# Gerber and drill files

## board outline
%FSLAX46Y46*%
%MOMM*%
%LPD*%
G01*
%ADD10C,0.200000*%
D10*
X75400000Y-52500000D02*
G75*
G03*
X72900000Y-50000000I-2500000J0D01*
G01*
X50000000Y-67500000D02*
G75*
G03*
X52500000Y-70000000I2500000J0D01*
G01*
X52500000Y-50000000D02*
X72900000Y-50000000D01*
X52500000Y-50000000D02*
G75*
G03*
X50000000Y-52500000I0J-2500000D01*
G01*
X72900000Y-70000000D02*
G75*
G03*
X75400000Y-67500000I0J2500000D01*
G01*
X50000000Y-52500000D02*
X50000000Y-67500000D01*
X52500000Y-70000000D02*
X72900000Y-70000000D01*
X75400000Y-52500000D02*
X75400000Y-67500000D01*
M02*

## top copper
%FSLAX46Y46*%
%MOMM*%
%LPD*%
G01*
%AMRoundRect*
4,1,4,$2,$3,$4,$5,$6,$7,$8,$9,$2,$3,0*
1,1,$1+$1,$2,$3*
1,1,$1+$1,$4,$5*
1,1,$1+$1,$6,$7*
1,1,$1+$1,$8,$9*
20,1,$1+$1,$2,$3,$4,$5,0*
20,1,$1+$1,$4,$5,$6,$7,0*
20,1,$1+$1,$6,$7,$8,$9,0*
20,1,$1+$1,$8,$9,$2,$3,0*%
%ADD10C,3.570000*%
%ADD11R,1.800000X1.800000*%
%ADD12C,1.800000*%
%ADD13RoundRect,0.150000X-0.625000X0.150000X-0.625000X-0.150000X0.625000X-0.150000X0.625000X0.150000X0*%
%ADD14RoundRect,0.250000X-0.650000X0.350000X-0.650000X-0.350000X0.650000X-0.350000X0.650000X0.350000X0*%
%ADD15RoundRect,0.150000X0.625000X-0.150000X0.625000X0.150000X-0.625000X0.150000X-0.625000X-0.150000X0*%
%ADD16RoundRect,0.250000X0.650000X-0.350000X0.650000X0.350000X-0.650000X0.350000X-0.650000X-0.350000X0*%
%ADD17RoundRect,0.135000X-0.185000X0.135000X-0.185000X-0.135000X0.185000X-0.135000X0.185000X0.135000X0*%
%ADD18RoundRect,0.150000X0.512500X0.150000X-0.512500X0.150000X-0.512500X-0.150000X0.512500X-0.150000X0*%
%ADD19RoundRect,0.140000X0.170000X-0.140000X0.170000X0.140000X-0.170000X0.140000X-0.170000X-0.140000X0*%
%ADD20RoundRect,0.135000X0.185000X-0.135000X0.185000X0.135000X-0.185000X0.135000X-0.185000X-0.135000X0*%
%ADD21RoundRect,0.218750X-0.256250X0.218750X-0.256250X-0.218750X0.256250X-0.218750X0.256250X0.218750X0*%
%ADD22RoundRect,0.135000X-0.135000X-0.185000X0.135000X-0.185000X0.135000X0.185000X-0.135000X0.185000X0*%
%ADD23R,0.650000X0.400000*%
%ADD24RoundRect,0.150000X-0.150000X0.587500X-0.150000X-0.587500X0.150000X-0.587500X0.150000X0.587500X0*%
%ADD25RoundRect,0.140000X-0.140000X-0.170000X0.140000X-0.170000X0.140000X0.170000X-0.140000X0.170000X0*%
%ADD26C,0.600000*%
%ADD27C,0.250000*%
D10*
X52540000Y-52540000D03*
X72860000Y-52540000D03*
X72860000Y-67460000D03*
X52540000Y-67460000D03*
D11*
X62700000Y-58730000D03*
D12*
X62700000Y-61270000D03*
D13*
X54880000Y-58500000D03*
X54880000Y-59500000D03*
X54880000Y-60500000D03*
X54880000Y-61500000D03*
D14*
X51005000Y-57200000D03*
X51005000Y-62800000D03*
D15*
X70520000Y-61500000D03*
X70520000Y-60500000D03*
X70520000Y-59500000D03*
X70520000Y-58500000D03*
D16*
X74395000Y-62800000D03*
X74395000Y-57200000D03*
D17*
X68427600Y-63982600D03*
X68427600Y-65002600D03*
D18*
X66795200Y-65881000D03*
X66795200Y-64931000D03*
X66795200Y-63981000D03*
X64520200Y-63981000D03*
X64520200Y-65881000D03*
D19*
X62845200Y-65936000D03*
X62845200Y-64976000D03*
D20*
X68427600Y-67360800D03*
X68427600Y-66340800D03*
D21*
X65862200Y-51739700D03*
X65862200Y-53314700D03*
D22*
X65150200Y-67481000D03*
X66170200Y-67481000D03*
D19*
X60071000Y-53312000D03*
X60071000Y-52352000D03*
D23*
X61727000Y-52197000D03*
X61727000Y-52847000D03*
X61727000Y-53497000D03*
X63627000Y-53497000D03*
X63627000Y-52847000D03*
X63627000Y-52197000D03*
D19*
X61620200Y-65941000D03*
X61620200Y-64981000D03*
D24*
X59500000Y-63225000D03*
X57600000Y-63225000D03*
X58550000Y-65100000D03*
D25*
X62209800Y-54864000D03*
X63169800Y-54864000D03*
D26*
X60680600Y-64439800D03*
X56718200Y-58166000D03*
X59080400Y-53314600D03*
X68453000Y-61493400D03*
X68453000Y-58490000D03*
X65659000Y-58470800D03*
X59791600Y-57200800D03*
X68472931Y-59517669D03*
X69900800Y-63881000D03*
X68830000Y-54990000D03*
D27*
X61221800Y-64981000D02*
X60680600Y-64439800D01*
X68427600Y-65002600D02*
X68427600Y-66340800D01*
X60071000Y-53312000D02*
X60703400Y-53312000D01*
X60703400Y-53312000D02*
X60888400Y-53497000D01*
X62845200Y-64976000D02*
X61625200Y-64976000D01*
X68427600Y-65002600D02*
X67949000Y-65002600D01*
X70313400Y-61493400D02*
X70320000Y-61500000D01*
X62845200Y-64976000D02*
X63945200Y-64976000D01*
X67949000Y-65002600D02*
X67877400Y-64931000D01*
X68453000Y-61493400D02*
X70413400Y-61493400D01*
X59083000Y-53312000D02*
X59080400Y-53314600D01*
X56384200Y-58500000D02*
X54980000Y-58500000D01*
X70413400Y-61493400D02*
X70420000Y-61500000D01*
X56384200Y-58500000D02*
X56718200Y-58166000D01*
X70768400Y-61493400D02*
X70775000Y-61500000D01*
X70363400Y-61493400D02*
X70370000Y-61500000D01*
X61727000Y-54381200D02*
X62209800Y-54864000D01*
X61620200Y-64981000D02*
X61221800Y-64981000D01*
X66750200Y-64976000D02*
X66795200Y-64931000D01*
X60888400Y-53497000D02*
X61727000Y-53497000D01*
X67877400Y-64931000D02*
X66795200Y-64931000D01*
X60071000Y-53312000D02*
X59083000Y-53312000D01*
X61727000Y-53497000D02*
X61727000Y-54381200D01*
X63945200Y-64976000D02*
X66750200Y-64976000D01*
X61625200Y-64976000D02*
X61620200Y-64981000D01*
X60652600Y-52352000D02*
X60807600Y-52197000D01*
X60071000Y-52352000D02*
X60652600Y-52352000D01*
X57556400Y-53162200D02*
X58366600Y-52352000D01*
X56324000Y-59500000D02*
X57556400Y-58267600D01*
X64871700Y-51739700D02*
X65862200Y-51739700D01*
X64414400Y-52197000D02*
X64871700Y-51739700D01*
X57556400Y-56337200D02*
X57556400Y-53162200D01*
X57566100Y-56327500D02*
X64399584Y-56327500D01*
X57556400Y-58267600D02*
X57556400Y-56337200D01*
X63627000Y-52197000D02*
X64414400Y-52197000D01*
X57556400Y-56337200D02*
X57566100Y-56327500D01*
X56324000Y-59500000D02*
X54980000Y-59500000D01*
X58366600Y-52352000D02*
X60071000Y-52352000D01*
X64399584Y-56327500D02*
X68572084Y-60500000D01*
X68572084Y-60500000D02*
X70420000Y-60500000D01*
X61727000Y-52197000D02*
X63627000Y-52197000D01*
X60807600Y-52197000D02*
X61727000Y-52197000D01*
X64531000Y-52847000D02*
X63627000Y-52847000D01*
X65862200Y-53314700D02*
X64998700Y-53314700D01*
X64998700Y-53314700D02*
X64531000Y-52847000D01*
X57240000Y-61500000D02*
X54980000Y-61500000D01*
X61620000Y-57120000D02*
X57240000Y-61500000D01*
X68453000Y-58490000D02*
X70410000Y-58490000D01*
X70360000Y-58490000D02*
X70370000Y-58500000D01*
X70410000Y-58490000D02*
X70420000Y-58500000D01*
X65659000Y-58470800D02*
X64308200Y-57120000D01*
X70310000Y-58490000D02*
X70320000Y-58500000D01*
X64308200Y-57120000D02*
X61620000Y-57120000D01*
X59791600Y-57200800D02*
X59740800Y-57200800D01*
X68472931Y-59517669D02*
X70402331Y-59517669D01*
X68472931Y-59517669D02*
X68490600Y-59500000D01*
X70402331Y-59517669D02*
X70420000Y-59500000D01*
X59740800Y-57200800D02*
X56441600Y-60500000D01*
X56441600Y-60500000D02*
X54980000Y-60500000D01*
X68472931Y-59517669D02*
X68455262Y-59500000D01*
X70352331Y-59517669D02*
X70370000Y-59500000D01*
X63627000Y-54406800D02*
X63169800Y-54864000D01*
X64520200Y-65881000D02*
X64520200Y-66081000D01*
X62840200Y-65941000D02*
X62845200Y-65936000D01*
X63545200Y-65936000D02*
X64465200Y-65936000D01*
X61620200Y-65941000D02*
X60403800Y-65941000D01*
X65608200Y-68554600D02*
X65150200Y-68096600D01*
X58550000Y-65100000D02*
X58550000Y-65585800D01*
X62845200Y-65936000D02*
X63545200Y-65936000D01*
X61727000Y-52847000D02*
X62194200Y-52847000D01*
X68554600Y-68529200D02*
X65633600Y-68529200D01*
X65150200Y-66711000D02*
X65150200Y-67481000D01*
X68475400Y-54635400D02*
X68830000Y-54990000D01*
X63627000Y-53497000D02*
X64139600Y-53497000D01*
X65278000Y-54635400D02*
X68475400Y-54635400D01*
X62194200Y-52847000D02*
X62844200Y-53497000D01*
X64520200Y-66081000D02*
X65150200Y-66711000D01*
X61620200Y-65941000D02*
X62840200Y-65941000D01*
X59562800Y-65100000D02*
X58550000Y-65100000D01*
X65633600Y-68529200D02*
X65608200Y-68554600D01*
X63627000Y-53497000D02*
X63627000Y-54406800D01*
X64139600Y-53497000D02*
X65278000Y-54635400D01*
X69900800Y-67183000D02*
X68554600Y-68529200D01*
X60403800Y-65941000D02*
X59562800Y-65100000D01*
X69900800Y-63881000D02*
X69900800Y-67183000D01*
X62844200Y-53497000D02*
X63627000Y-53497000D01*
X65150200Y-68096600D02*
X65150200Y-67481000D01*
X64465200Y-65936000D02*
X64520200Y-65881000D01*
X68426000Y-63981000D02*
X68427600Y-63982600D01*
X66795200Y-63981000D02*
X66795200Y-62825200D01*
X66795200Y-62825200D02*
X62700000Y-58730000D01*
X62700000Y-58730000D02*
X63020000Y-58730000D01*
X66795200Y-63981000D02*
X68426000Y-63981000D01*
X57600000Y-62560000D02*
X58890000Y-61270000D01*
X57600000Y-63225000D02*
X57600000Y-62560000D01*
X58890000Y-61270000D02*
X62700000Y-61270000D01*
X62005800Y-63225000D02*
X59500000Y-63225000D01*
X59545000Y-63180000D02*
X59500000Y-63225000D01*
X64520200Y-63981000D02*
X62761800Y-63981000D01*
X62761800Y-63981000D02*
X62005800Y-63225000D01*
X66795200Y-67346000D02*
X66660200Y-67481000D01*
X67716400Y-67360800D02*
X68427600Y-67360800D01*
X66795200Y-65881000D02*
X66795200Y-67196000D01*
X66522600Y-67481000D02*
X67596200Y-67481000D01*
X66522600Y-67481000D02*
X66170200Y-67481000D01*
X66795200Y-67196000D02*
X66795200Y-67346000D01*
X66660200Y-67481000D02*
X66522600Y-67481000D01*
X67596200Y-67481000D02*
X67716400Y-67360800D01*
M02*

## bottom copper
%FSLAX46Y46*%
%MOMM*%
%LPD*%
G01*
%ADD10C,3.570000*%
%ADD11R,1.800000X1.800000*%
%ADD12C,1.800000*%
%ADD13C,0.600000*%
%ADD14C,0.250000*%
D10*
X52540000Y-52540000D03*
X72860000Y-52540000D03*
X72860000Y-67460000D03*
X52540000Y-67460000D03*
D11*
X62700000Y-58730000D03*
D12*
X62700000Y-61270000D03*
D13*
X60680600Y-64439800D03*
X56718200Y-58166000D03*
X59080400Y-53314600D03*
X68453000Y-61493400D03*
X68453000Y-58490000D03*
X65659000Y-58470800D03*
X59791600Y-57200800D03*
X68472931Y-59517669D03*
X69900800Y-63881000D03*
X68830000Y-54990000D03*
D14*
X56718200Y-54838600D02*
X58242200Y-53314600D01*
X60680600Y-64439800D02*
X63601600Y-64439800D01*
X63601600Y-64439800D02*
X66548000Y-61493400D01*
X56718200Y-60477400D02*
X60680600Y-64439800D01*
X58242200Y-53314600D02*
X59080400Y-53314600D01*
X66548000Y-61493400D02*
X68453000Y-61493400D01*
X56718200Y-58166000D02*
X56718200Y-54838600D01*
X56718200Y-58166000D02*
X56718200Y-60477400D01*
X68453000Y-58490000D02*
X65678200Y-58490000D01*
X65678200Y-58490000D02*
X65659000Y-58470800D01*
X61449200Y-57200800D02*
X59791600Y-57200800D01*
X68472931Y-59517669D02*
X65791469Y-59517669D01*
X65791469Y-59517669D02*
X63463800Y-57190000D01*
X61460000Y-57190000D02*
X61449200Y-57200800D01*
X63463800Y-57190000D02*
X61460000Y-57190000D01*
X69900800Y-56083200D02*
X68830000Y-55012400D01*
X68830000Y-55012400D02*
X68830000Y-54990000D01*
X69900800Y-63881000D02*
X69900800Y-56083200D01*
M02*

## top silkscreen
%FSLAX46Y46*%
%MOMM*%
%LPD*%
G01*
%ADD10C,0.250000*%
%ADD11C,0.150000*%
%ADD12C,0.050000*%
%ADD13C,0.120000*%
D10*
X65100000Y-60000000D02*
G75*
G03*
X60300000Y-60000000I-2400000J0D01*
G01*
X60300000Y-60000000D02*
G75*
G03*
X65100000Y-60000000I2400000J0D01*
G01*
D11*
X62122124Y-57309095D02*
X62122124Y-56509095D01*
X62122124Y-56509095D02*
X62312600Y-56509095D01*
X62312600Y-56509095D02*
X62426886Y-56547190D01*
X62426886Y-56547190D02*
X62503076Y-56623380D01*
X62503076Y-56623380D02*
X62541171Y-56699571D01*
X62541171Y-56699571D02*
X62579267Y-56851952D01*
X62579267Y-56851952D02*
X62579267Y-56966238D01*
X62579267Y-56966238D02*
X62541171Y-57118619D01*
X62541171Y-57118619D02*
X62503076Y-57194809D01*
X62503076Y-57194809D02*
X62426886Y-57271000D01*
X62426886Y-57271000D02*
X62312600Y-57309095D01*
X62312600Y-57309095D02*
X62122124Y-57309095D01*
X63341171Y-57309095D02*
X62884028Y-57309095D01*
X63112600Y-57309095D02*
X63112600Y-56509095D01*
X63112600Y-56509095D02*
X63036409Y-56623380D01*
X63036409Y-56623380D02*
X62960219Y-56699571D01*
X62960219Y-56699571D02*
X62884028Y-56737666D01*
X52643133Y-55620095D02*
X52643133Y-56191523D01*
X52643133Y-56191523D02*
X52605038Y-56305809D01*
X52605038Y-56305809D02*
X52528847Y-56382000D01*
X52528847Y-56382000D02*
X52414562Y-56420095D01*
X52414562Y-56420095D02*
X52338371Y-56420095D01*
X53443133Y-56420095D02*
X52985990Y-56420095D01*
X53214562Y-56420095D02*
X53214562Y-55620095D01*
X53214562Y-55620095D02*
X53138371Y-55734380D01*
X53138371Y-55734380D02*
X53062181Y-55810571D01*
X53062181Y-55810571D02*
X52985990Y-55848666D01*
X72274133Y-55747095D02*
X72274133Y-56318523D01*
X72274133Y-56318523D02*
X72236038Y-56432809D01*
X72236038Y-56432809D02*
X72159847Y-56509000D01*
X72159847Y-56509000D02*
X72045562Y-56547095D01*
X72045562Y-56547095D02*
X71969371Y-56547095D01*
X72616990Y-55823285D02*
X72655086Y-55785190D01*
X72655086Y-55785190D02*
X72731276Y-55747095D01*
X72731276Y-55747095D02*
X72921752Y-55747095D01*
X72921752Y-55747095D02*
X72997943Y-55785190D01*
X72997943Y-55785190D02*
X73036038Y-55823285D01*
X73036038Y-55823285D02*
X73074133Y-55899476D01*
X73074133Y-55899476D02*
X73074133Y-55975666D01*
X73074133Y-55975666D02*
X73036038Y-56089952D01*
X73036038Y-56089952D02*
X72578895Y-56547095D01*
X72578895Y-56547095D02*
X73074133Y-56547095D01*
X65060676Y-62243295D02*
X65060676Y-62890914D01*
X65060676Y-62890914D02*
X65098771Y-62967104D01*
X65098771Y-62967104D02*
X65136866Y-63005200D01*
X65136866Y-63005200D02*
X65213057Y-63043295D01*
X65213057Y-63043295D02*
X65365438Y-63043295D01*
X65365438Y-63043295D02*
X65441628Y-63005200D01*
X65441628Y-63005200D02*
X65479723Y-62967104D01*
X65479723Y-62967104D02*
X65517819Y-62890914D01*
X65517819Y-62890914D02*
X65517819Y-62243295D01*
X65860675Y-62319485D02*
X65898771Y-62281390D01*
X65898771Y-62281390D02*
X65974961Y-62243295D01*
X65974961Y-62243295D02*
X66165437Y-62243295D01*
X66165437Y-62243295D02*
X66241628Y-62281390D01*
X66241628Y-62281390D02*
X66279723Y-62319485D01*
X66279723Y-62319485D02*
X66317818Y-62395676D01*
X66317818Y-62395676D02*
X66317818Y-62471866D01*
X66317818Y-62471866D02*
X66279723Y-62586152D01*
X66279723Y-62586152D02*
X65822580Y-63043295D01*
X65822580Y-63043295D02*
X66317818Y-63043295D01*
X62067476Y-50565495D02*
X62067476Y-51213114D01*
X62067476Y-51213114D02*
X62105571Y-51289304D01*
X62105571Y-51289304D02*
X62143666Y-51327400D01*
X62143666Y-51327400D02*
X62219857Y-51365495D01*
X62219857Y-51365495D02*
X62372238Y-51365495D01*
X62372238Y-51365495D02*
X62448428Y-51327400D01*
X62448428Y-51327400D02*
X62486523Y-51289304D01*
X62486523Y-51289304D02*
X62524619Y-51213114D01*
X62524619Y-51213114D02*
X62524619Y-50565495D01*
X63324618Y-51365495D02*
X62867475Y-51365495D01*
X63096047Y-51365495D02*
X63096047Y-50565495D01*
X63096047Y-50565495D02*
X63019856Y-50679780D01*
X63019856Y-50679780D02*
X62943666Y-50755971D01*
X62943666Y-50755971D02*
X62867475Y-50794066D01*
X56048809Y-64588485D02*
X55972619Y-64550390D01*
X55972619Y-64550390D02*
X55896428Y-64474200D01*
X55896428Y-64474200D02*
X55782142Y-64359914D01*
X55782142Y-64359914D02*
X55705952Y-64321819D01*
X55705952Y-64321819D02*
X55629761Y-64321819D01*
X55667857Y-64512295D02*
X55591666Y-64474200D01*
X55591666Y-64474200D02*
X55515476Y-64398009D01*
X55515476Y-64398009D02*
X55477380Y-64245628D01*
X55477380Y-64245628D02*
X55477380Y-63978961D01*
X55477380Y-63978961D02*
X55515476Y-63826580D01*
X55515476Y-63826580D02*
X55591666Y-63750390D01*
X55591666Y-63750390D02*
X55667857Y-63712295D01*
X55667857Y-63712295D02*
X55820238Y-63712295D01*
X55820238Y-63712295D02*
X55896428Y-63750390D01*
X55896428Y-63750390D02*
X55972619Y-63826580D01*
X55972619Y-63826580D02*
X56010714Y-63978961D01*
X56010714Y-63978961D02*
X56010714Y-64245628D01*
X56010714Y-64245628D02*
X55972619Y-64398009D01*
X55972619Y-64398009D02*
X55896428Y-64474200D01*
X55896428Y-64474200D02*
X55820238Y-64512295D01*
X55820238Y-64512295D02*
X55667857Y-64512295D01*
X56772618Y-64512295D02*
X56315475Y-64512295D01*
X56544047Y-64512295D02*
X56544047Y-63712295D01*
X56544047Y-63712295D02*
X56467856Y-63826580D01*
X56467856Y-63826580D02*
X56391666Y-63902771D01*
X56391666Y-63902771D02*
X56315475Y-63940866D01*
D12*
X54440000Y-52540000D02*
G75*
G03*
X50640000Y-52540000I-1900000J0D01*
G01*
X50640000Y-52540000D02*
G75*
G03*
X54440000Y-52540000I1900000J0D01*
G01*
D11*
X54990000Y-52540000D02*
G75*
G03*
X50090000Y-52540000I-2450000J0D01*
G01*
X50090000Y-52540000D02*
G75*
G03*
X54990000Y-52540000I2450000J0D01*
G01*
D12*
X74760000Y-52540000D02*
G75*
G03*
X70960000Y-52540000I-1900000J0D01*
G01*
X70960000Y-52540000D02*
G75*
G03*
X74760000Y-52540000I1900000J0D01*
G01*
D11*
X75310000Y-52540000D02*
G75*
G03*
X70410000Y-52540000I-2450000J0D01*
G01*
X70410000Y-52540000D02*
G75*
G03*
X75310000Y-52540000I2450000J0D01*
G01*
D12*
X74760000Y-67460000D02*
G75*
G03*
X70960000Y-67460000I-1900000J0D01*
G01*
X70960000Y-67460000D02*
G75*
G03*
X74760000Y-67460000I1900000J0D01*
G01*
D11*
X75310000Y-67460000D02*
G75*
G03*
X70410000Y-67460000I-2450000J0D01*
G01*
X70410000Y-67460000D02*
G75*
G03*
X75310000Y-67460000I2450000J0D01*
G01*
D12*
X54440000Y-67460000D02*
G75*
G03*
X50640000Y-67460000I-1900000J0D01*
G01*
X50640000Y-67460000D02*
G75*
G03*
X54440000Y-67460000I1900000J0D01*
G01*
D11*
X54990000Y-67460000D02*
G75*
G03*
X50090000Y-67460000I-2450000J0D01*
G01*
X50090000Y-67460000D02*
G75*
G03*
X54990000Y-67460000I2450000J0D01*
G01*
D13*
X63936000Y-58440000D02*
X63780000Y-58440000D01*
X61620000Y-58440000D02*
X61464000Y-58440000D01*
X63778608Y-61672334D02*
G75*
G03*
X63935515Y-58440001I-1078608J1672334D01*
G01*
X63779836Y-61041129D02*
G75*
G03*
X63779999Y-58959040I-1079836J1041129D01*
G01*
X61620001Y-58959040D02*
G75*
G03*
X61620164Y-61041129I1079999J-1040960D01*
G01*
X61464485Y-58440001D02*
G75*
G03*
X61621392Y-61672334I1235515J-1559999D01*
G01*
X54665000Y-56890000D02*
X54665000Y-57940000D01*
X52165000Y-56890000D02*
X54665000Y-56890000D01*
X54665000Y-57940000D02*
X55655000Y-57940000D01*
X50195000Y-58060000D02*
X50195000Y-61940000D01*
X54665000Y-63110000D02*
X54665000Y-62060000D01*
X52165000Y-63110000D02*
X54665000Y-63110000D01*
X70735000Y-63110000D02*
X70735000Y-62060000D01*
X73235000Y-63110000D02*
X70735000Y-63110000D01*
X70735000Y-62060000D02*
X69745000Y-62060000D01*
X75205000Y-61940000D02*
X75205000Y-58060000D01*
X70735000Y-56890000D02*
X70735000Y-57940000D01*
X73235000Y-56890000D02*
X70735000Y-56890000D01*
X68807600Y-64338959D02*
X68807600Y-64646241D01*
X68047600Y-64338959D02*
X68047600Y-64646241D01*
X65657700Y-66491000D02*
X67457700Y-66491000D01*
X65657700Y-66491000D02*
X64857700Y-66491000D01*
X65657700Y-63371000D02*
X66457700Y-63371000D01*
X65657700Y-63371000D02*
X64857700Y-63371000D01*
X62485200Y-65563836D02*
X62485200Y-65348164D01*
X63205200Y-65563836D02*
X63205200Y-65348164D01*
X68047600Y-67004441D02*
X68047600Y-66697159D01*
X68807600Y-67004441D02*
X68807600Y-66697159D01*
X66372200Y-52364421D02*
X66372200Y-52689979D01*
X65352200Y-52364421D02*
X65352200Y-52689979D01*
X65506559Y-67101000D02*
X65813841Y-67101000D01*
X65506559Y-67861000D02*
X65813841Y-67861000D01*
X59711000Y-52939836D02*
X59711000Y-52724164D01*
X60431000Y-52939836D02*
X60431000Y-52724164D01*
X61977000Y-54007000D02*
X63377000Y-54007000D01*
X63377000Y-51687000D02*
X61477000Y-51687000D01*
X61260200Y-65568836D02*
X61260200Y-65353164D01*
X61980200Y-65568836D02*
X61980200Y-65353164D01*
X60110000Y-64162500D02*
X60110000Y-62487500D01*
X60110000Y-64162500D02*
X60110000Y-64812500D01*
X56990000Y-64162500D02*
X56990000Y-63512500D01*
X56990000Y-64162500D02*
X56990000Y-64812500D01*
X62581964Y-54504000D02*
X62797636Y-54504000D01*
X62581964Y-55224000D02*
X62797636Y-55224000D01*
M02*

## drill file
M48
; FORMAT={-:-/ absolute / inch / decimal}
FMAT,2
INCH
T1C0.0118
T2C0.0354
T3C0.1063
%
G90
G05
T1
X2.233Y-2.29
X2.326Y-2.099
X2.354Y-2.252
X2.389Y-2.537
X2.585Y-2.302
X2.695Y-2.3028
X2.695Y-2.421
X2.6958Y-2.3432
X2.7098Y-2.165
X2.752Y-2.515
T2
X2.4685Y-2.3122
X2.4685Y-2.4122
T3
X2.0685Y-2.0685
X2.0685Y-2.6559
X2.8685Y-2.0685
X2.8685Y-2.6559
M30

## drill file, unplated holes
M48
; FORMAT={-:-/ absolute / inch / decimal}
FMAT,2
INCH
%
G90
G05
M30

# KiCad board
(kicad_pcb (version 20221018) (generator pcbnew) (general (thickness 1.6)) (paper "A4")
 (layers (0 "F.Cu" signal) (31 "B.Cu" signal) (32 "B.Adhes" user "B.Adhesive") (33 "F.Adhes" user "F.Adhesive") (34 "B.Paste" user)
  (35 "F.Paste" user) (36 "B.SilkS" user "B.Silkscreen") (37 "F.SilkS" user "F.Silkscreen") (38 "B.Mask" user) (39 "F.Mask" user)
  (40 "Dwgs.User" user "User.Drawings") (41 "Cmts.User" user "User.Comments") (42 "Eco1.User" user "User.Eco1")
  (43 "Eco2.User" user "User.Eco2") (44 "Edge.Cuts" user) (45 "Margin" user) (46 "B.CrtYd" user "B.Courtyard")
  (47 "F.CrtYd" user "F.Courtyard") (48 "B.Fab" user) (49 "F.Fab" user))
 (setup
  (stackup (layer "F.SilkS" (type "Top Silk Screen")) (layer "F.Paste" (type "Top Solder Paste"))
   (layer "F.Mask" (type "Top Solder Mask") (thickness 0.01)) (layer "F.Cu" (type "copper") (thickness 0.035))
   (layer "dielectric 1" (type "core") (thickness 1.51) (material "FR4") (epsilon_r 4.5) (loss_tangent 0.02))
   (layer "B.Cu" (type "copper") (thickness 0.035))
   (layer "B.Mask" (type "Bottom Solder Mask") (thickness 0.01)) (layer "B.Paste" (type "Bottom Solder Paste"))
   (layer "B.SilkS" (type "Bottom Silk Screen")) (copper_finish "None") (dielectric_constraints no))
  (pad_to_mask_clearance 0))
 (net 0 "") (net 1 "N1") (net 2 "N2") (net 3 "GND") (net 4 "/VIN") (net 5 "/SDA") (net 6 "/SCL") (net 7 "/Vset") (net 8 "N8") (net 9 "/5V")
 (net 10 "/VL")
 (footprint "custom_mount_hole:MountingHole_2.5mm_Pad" (layer "F.Cu") (at 52.54 52.54)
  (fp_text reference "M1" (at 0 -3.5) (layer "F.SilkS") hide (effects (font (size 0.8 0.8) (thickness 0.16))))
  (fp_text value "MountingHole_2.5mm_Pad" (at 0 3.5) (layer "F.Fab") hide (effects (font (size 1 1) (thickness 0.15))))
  (fp_circle (center 0 0) (end 1.9 0) (stroke (width 0.05) (type solid)) (fill none) (layer "F.SilkS"))
  (fp_circle (center 0 0) (end 2.45 0) (stroke (width 0.15) (type solid)) (fill none) (layer "F.SilkS"))
  (pad "~" thru_hole circle (at 0 0) (size 3.57 3.57) (drill 2.7) (layers "*.Cu" "*.Mask")))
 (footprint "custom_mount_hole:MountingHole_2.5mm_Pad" (layer "F.Cu") (at 72.86 52.54)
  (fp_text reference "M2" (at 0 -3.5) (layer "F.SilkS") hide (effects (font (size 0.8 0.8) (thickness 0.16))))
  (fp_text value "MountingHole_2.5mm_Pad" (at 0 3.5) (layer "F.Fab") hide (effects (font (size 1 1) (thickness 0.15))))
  (fp_circle (center 0 0) (end 1.9 0) (stroke (width 0.05) (type solid)) (fill none) (layer "F.SilkS"))
  (fp_circle (center 0 0) (end 2.45 0) (stroke (width 0.15) (type solid)) (fill none) (layer "F.SilkS"))
  (pad "~" thru_hole circle (at 0 0) (size 3.57 3.57) (drill 2.7) (layers "*.Cu" "*.Mask")))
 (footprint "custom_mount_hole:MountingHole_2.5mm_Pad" (layer "F.Cu") (at 72.86 67.46)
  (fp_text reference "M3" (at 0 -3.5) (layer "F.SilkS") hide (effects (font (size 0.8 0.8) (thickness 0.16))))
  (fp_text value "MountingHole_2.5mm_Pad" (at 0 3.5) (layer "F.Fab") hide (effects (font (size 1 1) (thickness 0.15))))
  (fp_circle (center 0 0) (end 1.9 0) (stroke (width 0.05) (type solid)) (fill none) (layer "F.SilkS"))
  (fp_circle (center 0 0) (end 2.45 0) (stroke (width 0.15) (type solid)) (fill none) (layer "F.SilkS"))
  (pad "~" thru_hole circle (at 0 0) (size 3.57 3.57) (drill 2.7) (layers "*.Cu" "*.Mask")))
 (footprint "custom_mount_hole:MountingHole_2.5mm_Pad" (layer "F.Cu") (at 52.54 67.46)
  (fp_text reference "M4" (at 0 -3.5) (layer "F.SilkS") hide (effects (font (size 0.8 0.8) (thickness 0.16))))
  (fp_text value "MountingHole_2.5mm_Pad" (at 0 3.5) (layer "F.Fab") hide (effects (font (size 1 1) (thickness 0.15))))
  (fp_circle (center 0 0) (end 1.9 0) (stroke (width 0.05) (type solid)) (fill none) (layer "F.SilkS"))
  (fp_circle (center 0 0) (end 2.45 0) (stroke (width 0.15) (type solid)) (fill none) (layer "F.SilkS"))
  (pad "~" thru_hole circle (at 0 0) (size 3.57 3.57) (drill 2.7) (layers "*.Cu" "*.Mask")))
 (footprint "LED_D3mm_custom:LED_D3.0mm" (layer "F.Cu") (at 62.7 58.73 -90)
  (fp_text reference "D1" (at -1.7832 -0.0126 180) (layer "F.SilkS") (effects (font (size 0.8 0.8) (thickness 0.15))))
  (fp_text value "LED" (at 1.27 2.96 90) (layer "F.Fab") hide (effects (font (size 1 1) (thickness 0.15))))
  (fp_line (start -0.29 -1.236) (end -0.29 -1.08) (stroke (width 0.12) (type solid)) (layer "F.SilkS"))
  (fp_line (start -0.29 1.08) (end -0.29 1.236) (stroke (width 0.12) (type solid)) (layer "F.SilkS"))
  (fp_arc (start -0.29 -1.235516) (mid 1.366487 -1.987659) (end 2.942335 -1.078608) (stroke (width 0.12) (type solid)) (layer "F.SilkS"))
  (fp_arc (start 0.229039 -1.08) (mid 1.270117 -1.5) (end 2.31113 -1.079837) (stroke (width 0.12) (type solid)) (layer "F.SilkS"))
  (fp_arc (start 2.31113 1.079837) (mid 1.270117 1.5) (end 0.229039 1.08) (stroke (width 0.12) (type solid)) (layer "F.SilkS"))
  (fp_arc (start 2.942335 1.078608) (mid 1.366487 1.987659) (end -0.29 1.235516) (stroke (width 0.12) (type solid)) (layer "F.SilkS"))
  (pad "1" thru_hole rect (at 0 0 270) (size 1.8 1.8) (drill 0.9) (layers "*.Cu" "*.Mask") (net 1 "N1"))
  (pad "2" thru_hole circle (at 2.54 0 270) (size 1.8 1.8) (drill 0.9) (layers "*.Cu" "*.Mask") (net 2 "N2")))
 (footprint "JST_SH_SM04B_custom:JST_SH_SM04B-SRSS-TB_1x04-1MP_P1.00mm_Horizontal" (layer "F.Cu") (at 52.88 60 -90)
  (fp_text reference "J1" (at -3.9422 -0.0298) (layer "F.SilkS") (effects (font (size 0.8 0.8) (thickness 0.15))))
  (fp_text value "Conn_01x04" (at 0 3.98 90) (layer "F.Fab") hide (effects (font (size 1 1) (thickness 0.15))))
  (fp_line (start -3.11 -1.785) (end -2.06 -1.785) (stroke (width 0.12) (type solid)) (layer "F.SilkS"))
  (fp_line (start -3.11 0.715) (end -3.11 -1.785) (stroke (width 0.12) (type solid)) (layer "F.SilkS"))
  (fp_line (start -2.06 -1.785) (end -2.06 -2.775) (stroke (width 0.12) (type solid)) (layer "F.SilkS"))
  (fp_line (start -1.94 2.685) (end 1.94 2.685) (stroke (width 0.12) (type solid)) (layer "F.SilkS"))
  (fp_line (start 3.11 -1.785) (end 2.06 -1.785) (stroke (width 0.12) (type solid)) (layer "F.SilkS"))
  (fp_line (start 3.11 0.715) (end 3.11 -1.785) (stroke (width 0.12) (type solid)) (layer "F.SilkS"))
  (pad "1" smd roundrect (at -1.5 -2 270) (size 0.6 1.55) (layers "F.Cu" "F.Paste" "F.Mask") (roundrect_rratio 0.25) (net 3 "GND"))
  (pad "2" smd roundrect (at -0.5 -2 270) (size 0.6 1.55) (layers "F.Cu" "F.Paste" "F.Mask") (roundrect_rratio 0.25) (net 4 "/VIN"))
  (pad "3" smd roundrect (at 0.5 -2 270) (size 0.6 1.55) (layers "F.Cu" "F.Paste" "F.Mask") (roundrect_rratio 0.25) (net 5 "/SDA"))
  (pad "4" smd roundrect (at 1.5 -2 270) (size 0.6 1.55) (layers "F.Cu" "F.Paste" "F.Mask") (roundrect_rratio 0.25) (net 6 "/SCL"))
  (pad "MP" smd roundrect (at -2.8 1.875 270) (size 1.2 1.8) (layers "F.Cu" "F.Paste" "F.Mask") (roundrect_rratio 0.2083333333))
  (pad "MP" smd roundrect (at 2.8 1.875 270) (size 1.2 1.8) (layers "F.Cu" "F.Paste" "F.Mask") (roundrect_rratio 0.2083333333)))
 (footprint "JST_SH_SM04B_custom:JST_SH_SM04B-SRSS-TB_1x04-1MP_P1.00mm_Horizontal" (layer "F.Cu") (at 72.52 60 90)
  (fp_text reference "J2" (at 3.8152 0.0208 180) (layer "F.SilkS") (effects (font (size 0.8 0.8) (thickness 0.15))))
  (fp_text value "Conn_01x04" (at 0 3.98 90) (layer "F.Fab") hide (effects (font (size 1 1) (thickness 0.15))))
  (fp_line (start -3.11 -1.785) (end -2.06 -1.785) (stroke (width 0.12) (type solid)) (layer "F.SilkS"))
  (fp_line (start -3.11 0.715) (end -3.11 -1.785) (stroke (width 0.12) (type solid)) (layer "F.SilkS"))
  (fp_line (start -2.06 -1.785) (end -2.06 -2.775) (stroke (width 0.12) (type solid)) (layer "F.SilkS"))
  (fp_line (start -1.94 2.685) (end 1.94 2.685) (stroke (width 0.12) (type solid)) (layer "F.SilkS"))
  (fp_line (start 3.11 -1.785) (end 2.06 -1.785) (stroke (width 0.12) (type solid)) (layer "F.SilkS"))
  (fp_line (start 3.11 0.715) (end 3.11 -1.785) (stroke (width 0.12) (type solid)) (layer "F.SilkS"))
  (pad "1" smd roundrect (at -1.5 -2 90) (size 0.6 1.55) (layers "F.Cu" "F.Paste" "F.Mask") (roundrect_rratio 0.25) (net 3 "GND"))
  (pad "2" smd roundrect (at -0.5 -2 90) (size 0.6 1.55) (layers "F.Cu" "F.Paste" "F.Mask") (roundrect_rratio 0.25) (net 4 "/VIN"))
  (pad "3" smd roundrect (at 0.5 -2 90) (size 0.6 1.55) (layers "F.Cu" "F.Paste" "F.Mask") (roundrect_rratio 0.25) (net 5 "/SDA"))
  (pad "4" smd roundrect (at 1.5 -2 90) (size 0.6 1.55) (layers "F.Cu" "F.Paste" "F.Mask") (roundrect_rratio 0.25) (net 6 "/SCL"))
  (pad "MP" smd roundrect (at -2.8 1.875 90) (size 1.2 1.8) (layers "F.Cu" "F.Paste" "F.Mask") (roundrect_rratio 0.2083333333))
  (pad "MP" smd roundrect (at 2.8 1.875 90) (size 1.2 1.8) (layers "F.Cu" "F.Paste" "F.Mask") (roundrect_rratio 0.2083333333)))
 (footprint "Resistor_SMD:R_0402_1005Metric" (layer "F.Cu") (at 68.4276 64.4926 -90)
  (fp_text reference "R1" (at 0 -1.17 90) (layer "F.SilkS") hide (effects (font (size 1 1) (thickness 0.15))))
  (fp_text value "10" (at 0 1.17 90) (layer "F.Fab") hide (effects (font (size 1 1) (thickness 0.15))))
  (fp_line (start -0.153641 -0.38) (end 0.153641 -0.38) (stroke (width 0.12) (type solid)) (layer "F.SilkS"))
  (fp_line (start -0.153641 0.38) (end 0.153641 0.38) (stroke (width 0.12) (type solid)) (layer "F.SilkS"))
  (pad "1" smd roundrect (at -0.51 0 270) (size 0.54 0.64) (layers "F.Cu" "F.Paste" "F.Mask") (roundrect_rratio 0.25) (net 1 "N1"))
  (pad "2" smd roundrect (at 0.51 0 270) (size 0.54 0.64) (layers "F.Cu" "F.Paste" "F.Mask") (roundrect_rratio 0.25) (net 3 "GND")))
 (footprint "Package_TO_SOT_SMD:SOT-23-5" (layer "F.Cu") (at 65.6577 64.931 180)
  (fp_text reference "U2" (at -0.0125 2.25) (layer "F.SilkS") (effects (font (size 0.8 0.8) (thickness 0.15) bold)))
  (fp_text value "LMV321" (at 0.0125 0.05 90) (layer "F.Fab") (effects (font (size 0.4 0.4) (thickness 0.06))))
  (fp_line (start 0 -1.56) (end -1.8 -1.56) (stroke (width 0.12) (type solid)) (layer "F.SilkS"))
  (fp_line (start 0 -1.56) (end 0.8 -1.56) (stroke (width 0.12) (type solid)) (layer "F.SilkS"))
  (fp_line (start 0 1.56) (end -0.8 1.56) (stroke (width 0.12) (type solid)) (layer "F.SilkS"))
  (fp_line (start 0 1.56) (end 0.8 1.56) (stroke (width 0.12) (type solid)) (layer "F.SilkS"))
  (pad "1" smd roundrect (at -1.1375 -0.95 180) (size 1.325 0.6) (layers "F.Cu" "F.Paste" "F.Mask") (roundrect_rratio 0.25) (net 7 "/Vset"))
  (pad "2" smd roundrect (at -1.1375 0 180) (size 1.325 0.6) (layers "F.Cu" "F.Paste" "F.Mask") (roundrect_rratio 0.25) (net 3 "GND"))
  (pad "3" smd roundrect (at -1.1375 0.95 180) (size 1.325 0.6) (layers "F.Cu" "F.Paste" "F.Mask") (roundrect_rratio 0.25) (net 1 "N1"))
  (pad "4" smd roundrect (at 1.1375 0.95 180) (size 1.325 0.6) (layers "F.Cu" "F.Paste" "F.Mask") (roundrect_rratio 0.25) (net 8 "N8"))
  (pad "5" smd roundrect (at 1.1375 -0.95 180) (size 1.325 0.6) (layers "F.Cu" "F.Paste" "F.Mask") (roundrect_rratio 0.25) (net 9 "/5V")))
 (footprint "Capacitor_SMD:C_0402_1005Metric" (layer "F.Cu") (at 62.8452 65.456 90)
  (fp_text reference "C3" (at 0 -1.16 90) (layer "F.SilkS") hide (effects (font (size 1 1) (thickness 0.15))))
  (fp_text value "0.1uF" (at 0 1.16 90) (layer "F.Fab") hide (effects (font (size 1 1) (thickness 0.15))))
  (fp_line (start -0.107836 -0.36) (end 0.107836 -0.36) (stroke (width 0.12) (type solid)) (layer "F.SilkS"))
  (fp_line (start -0.107836 0.36) (end 0.107836 0.36) (stroke (width 0.12) (type solid)) (layer "F.SilkS"))
  (pad "1" smd roundrect (at -0.48 0 90) (size 0.56 0.62) (layers "F.Cu" "F.Paste" "F.Mask") (roundrect_rratio 0.25) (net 9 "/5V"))
  (pad "2" smd roundrect (at 0.48 0 90) (size 0.56 0.62) (layers "F.Cu" "F.Paste" "F.Mask") (roundrect_rratio 0.25) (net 3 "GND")))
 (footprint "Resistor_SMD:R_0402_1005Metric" (layer "F.Cu") (at 68.4276 66.8508 90)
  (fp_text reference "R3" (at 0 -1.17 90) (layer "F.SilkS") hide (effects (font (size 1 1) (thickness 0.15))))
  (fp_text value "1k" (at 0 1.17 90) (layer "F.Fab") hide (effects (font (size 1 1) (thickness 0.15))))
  (fp_line (start -0.153641 -0.38) (end 0.153641 -0.38) (stroke (width 0.12) (type solid)) (layer "F.SilkS"))
  (fp_line (start -0.153641 0.38) (end 0.153641 0.38) (stroke (width 0.12) (type solid)) (layer "F.SilkS"))
  (pad "1" smd roundrect (at -0.51 0 90) (size 0.54 0.64) (layers "F.Cu" "F.Paste" "F.Mask") (roundrect_rratio 0.25) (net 7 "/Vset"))
  (pad "2" smd roundrect (at 0.51 0 90) (size 0.54 0.64) (layers "F.Cu" "F.Paste" "F.Mask") (roundrect_rratio 0.25) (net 3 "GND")))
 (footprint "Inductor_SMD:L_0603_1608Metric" (layer "F.Cu") (at 65.8622 52.5272 -90)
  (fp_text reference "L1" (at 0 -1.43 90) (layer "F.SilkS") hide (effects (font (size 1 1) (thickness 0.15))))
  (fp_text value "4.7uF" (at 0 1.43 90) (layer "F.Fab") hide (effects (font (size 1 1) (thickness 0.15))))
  (fp_line (start -0.162779 -0.51) (end 0.162779 -0.51) (stroke (width 0.12) (type solid)) (layer "F.SilkS"))
  (fp_line (start -0.162779 0.51) (end 0.162779 0.51) (stroke (width 0.12) (type solid)) (layer "F.SilkS"))
  (pad "1" smd roundrect (at -0.7875 0 270) (size 0.875 0.95) (layers "F.Cu" "F.Paste" "F.Mask") (roundrect_rratio 0.25) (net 4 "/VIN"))
  (pad "2" smd roundrect (at 0.7875 0 270) (size 0.875 0.95) (layers "F.Cu" "F.Paste" "F.Mask") (roundrect_rratio 0.25) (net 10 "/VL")))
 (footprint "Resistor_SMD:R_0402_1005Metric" (layer "F.Cu") (at 65.6602 67.481)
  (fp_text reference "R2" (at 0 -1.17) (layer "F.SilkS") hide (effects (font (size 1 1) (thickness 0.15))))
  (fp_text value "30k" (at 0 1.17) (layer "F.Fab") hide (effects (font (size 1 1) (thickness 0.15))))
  (fp_line (start -0.153641 -0.38) (end 0.153641 -0.38) (stroke (width 0.12) (type solid)) (layer "F.SilkS"))
  (fp_line (start -0.153641 0.38) (end 0.153641 0.38) (stroke (width 0.12) (type solid)) (layer "F.SilkS"))
  (pad "1" smd roundrect (at -0.51 0) (size 0.54 0.64) (layers "F.Cu" "F.Paste" "F.Mask") (roundrect_rratio 0.25) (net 9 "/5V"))
  (pad "2" smd roundrect (at 0.51 0) (size 0.54 0.64) (layers "F.Cu" "F.Paste" "F.Mask") (roundrect_rratio 0.25) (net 7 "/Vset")))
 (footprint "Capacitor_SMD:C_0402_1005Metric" (layer "F.Cu") (at 60.071 52.832 90)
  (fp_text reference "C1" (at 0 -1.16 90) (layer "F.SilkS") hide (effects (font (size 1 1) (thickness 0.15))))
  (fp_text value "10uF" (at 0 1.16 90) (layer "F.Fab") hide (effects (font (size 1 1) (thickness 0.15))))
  (fp_line (start -0.107836 -0.36) (end 0.107836 -0.36) (stroke (width 0.12) (type solid)) (layer "F.SilkS"))
  (fp_line (start -0.107836 0.36) (end 0.107836 0.36) (stroke (width 0.12) (type solid)) (layer "F.SilkS"))
  (pad "1" smd roundrect (at -0.48 0 90) (size 0.56 0.62) (layers "F.Cu" "F.Paste" "F.Mask") (roundrect_rratio 0.25) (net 3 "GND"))
  (pad "2" smd roundrect (at 0.48 0 90) (size 0.56 0.62) (layers "F.Cu" "F.Paste" "F.Mask") (roundrect_rratio 0.25) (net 4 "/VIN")))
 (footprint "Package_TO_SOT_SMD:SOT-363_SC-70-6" (layer "F.Cu") (at 62.677 52.847)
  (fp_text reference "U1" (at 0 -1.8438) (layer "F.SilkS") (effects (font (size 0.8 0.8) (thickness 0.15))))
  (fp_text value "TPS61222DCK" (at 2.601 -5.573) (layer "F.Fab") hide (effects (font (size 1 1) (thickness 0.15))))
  (fp_line (start -0.7 1.16) (end 0.7 1.16) (stroke (width 0.12) (type solid)) (layer "F.SilkS"))
  (fp_line (start 0.7 -1.16) (end -1.2 -1.16) (stroke (width 0.12) (type solid)) (layer "F.SilkS"))
  (pad "1" smd rect (at -0.95 -0.65) (size 0.65 0.4) (layers "F.Cu" "F.Paste" "F.Mask") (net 4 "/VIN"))
  (pad "2" smd rect (at -0.95 0) (size 0.65 0.4) (layers "F.Cu" "F.Paste" "F.Mask") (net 9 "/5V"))
  (pad "3" smd rect (at -0.95 0.65) (size 0.65 0.4) (layers "F.Cu" "F.Paste" "F.Mask") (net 3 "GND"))
  (pad "4" smd rect (at 0.95 0.65) (size 0.65 0.4) (layers "F.Cu" "F.Paste" "F.Mask") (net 9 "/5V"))
  (pad "5" smd rect (at 0.95 0) (size 0.65 0.4) (layers "F.Cu" "F.Paste" "F.Mask") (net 10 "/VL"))
  (pad "6" smd rect (at 0.95 -0.65) (size 0.65 0.4) (layers "F.Cu" "F.Paste" "F.Mask") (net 4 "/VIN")))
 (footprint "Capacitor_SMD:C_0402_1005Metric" (layer "F.Cu") (at 61.6202 65.461 90)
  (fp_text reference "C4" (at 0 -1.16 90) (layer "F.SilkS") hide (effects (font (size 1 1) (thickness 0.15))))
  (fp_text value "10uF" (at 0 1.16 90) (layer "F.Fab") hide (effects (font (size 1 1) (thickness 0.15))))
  (fp_line (start -0.107836 -0.36) (end 0.107836 -0.36) (stroke (width 0.12) (type solid)) (layer "F.SilkS"))
  (fp_line (start -0.107836 0.36) (end 0.107836 0.36) (stroke (width 0.12) (type solid)) (layer "F.SilkS"))
  (pad "1" smd roundrect (at -0.48 0 90) (size 0.56 0.62) (layers "F.Cu" "F.Paste" "F.Mask") (roundrect_rratio 0.25) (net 9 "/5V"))
  (pad "2" smd roundrect (at 0.48 0 90) (size 0.56 0.62) (layers "F.Cu" "F.Paste" "F.Mask") (roundrect_rratio 0.25) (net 3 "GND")))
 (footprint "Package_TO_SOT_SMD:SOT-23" (layer "F.Cu") (at 58.55 64.1625 -90)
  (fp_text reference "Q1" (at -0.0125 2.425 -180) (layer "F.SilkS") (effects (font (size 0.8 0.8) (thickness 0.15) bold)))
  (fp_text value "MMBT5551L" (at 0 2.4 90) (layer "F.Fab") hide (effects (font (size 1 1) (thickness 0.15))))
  (fp_line (start 0 -1.56) (end -1.675 -1.56) (stroke (width 0.12) (type solid)) (layer "F.SilkS"))
  (fp_line (start 0 -1.56) (end 0.65 -1.56) (stroke (width 0.12) (type solid)) (layer "F.SilkS"))
  (fp_line (start 0 1.56) (end -0.65 1.56) (stroke (width 0.12) (type solid)) (layer "F.SilkS"))
  (fp_line (start 0 1.56) (end 0.65 1.56) (stroke (width 0.12) (type solid)) (layer "F.SilkS"))
  (pad "1" smd roundrect (at -0.9375 -0.95 270) (size 1.475 0.6) (layers "F.Cu" "F.Paste" "F.Mask") (roundrect_rratio 0.25) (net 8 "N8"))
  (pad "2" smd roundrect (at -0.9375 0.95 270) (size 1.475 0.6) (layers "F.Cu" "F.Paste" "F.Mask") (roundrect_rratio 0.25) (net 2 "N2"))
  (pad "3" smd roundrect (at 0.9375 0 270) (size 1.475 0.6) (layers "F.Cu" "F.Paste" "F.Mask") (roundrect_rratio 0.25) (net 9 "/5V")))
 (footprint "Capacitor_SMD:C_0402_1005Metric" (layer "F.Cu") (at 62.6898 54.864)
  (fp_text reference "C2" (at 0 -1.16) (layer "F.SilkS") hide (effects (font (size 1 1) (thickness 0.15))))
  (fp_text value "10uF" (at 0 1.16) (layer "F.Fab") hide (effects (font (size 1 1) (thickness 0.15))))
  (fp_line (start -0.107836 -0.36) (end 0.107836 -0.36) (stroke (width 0.12) (type solid)) (layer "F.SilkS"))
  (fp_line (start -0.107836 0.36) (end 0.107836 0.36) (stroke (width 0.12) (type solid)) (layer "F.SilkS"))
  (pad "1" smd roundrect (at -0.48 0) (size 0.56 0.62) (layers "F.Cu" "F.Paste" "F.Mask") (roundrect_rratio 0.25) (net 3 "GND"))
  (pad "2" smd roundrect (at 0.48 0) (size 0.56 0.62) (layers "F.Cu" "F.Paste" "F.Mask") (roundrect_rratio 0.25) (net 9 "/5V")))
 (gr_circle (center 62.7 60) (end 65.1 60) (stroke (width 0.25) (type solid)) (fill none) (layer "F.SilkS"))
 (gr_arc (start 72.9 50) (mid 74.667767 50.732233) (end 75.4 52.5) (stroke (width 0.2) (type solid)) (layer "Edge.Cuts"))
 (gr_arc (start 52.5 70) (mid 50.732233 69.267767) (end 50 67.5) (stroke (width 0.2) (type solid)) (layer "Edge.Cuts"))
 (gr_line (start 52.5 50) (end 72.9 50) (stroke (width 0.2) (type solid)) (layer "Edge.Cuts"))
 (gr_arc (start 50 52.5) (mid 50.732233 50.732233) (end 52.5 50) (stroke (width 0.2) (type solid)) (layer "Edge.Cuts"))
 (gr_arc (start 75.4 67.5) (mid 74.667767 69.267767) (end 72.9 70) (stroke (width 0.2) (type solid)) (layer "Edge.Cuts"))
 (gr_line (start 50 52.5) (end 50 67.5) (stroke (width 0.2) (type solid)) (layer "Edge.Cuts"))
 (gr_line (start 52.5 70) (end 72.9 70) (stroke (width 0.2) (type solid)) (layer "Edge.Cuts"))
 (gr_line (start 75.4 52.5) (end 75.4 67.5) (stroke (width 0.2) (type solid)) (layer "Edge.Cuts"))
 (segment (start 61.2218 64.981) (end 60.6806 64.4398) (width 0.25) (layer "F.Cu") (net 3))
 (segment (start 68.4276 65.0026) (end 68.4276 66.3408) (width 0.25) (layer "F.Cu") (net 3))
 (segment (start 60.071 53.312) (end 60.7034 53.312) (width 0.25) (layer "F.Cu") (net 3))
 (segment (start 60.7034 53.312) (end 60.8884 53.497) (width 0.25) (layer "F.Cu") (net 3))
 (segment (start 62.8452 64.976) (end 61.6252 64.976) (width 0.25) (layer "F.Cu") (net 3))
 (segment (start 68.4276 65.0026) (end 67.949 65.0026) (width 0.25) (layer "F.Cu") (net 3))
 (segment (start 70.3134 61.4934) (end 70.32 61.5) (width 0.25) (layer "F.Cu") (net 3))
 (segment (start 62.8452 64.976) (end 63.9452 64.976) (width 0.25) (layer "F.Cu") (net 3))
 (segment (start 67.949 65.0026) (end 67.8774 64.931) (width 0.25) (layer "F.Cu") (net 3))
 (segment (start 68.453 61.4934) (end 70.4134 61.4934) (width 0.25) (layer "F.Cu") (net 3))
 (segment (start 59.083 53.312) (end 59.0804 53.3146) (width 0.25) (layer "F.Cu") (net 3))
 (segment (start 56.3842 58.5) (end 54.98 58.5) (width 0.25) (layer "F.Cu") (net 3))
 (segment (start 70.4134 61.4934) (end 70.42 61.5) (width 0.25) (layer "F.Cu") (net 3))
 (segment (start 56.3842 58.5) (end 56.7182 58.166) (width 0.25) (layer "F.Cu") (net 3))
 (segment (start 70.7684 61.4934) (end 70.775 61.5) (width 0.25) (layer "F.Cu") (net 3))
 (segment (start 70.3634 61.4934) (end 70.37 61.5) (width 0.25) (layer "F.Cu") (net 3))
 (segment (start 61.727 54.3812) (end 62.2098 54.864) (width 0.25) (layer "F.Cu") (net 3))
 (segment (start 61.6202 64.981) (end 61.2218 64.981) (width 0.25) (layer "F.Cu") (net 3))
 (segment (start 66.7502 64.976) (end 66.7952 64.931) (width 0.25) (layer "F.Cu") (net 3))
 (segment (start 60.8884 53.497) (end 61.727 53.497) (width 0.25) (layer "F.Cu") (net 3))
 (segment (start 67.8774 64.931) (end 66.7952 64.931) (width 0.25) (layer "F.Cu") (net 3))
 (segment (start 60.071 53.312) (end 59.083 53.312) (width 0.25) (layer "F.Cu") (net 3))
 (segment (start 61.727 53.497) (end 61.727 54.3812) (width 0.25) (layer "F.Cu") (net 3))
 (segment (start 63.9452 64.976) (end 66.7502 64.976) (width 0.25) (layer "F.Cu") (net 3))
 (segment (start 61.6252 64.976) (end 61.6202 64.981) (width 0.25) (layer "F.Cu") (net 3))
 (via (at 60.6806 64.4398) (size 0.6) (drill 0.3) (layers "F.Cu" "B.Cu") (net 3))
 (via (at 56.7182 58.166) (size 0.6) (drill 0.3) (layers "F.Cu" "B.Cu") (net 3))
 (via (at 59.0804 53.3146) (size 0.6) (drill 0.3) (layers "F.Cu" "B.Cu") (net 3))
 (via (at 68.453 61.4934) (size 0.6) (drill 0.3) (layers "F.Cu" "B.Cu") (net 3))
 (segment (start 56.7182 54.8386) (end 58.2422 53.3146) (width 0.25) (layer "B.Cu") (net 3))
 (segment (start 60.6806 64.4398) (end 63.6016 64.4398) (width 0.25) (layer "B.Cu") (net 3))
 (segment (start 63.6016 64.4398) (end 66.548 61.4934) (width 0.25) (layer "B.Cu") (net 3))
 (segment (start 56.7182 60.4774) (end 60.6806 64.4398) (width 0.25) (layer "B.Cu") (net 3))
 (segment (start 58.2422 53.3146) (end 59.0804 53.3146) (width 0.25) (layer "B.Cu") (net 3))
 (segment (start 66.548 61.4934) (end 68.453 61.4934) (width 0.25) (layer "B.Cu") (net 3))
 (segment (start 56.7182 58.166) (end 56.7182 54.8386) (width 0.25) (layer "B.Cu") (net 3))
 (segment (start 56.7182 58.166) (end 56.7182 60.4774) (width 0.25) (layer "B.Cu") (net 3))
 (segment (start 60.6526 52.352) (end 60.8076 52.197) (width 0.25) (layer "F.Cu") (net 4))
 (segment (start 60.071 52.352) (end 60.6526 52.352) (width 0.25) (layer "F.Cu") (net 4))
 (segment (start 57.5564 53.1622) (end 58.3666 52.352) (width 0.25) (layer "F.Cu") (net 4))
 (segment (start 56.324 59.5) (end 57.5564 58.2676) (width 0.25) (layer "F.Cu") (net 4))
 (segment (start 64.8717 51.7397) (end 65.8622 51.7397) (width 0.25) (layer "F.Cu") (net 4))
 (segment (start 64.4144 52.197) (end 64.8717 51.7397) (width 0.25) (layer "F.Cu") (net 4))
 (segment (start 57.5564 56.3372) (end 57.5564 53.1622) (width 0.25) (layer "F.Cu") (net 4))
 (segment (start 57.5661 56.3275) (end 64.399584 56.3275) (width 0.25) (layer "F.Cu") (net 4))
 (segment (start 57.5564 58.2676) (end 57.5564 56.3372) (width 0.25) (layer "F.Cu") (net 4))
 (segment (start 63.627 52.197) (end 64.4144 52.197) (width 0.25) (layer "F.Cu") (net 4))
 (segment (start 57.5564 56.3372) (end 57.5661 56.3275) (width 0.25) (layer "F.Cu") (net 4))
 (segment (start 56.324 59.5) (end 54.98 59.5) (width 0.25) (layer "F.Cu") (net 4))
 (segment (start 58.3666 52.352) (end 60.071 52.352) (width 0.25) (layer "F.Cu") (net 4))
 (segment (start 64.399584 56.3275) (end 68.572084 60.5) (width 0.25) (layer "F.Cu") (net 4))
 (segment (start 68.572084 60.5) (end 70.42 60.5) (width 0.25) (layer "F.Cu") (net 4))
 (segment (start 61.727 52.197) (end 63.627 52.197) (width 0.25) (layer "F.Cu") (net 4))
 (segment (start 60.8076 52.197) (end 61.727 52.197) (width 0.25) (layer "F.Cu") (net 4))
 (segment (start 64.531 52.847) (end 63.627 52.847) (width 0.25) (layer "F.Cu") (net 10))
 (segment (start 65.8622 53.3147) (end 64.9987 53.3147) (width 0.25) (layer "F.Cu") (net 10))
 (segment (start 64.9987 53.3147) (end 64.531 52.847) (width 0.25) (layer "F.Cu") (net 10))
 (segment (start 57.24 61.5) (end 54.98 61.5) (width 0.25) (layer "F.Cu") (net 6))
 (segment (start 61.62 57.12) (end 57.24 61.5) (width 0.25) (layer "F.Cu") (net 6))
 (segment (start 68.453 58.49) (end 70.41 58.49) (width 0.25) (layer "F.Cu") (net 6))
 (segment (start 70.36 58.49) (end 70.37 58.5) (width 0.25) (layer "F.Cu") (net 6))
 (segment (start 70.41 58.49) (end 70.42 58.5) (width 0.25) (layer "F.Cu") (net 6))
 (segment (start 65.659 58.4708) (end 64.3082 57.12) (width 0.25) (layer "F.Cu") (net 6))
 (segment (start 70.31 58.49) (end 70.32 58.5) (width 0.25) (layer "F.Cu") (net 6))
 (segment (start 64.3082 57.12) (end 61.62 57.12) (width 0.25) (layer "F.Cu") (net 6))
 (via (at 68.453 58.49) (size 0.6) (drill 0.3) (layers "F.Cu" "B.Cu") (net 6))
 (via (at 65.659 58.4708) (size 0.6) (drill 0.3) (layers "F.Cu" "B.Cu") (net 6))
 (segment (start 68.453 58.49) (end 65.6782 58.49) (width 0.25) (layer "B.Cu") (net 6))
 (segment (start 65.6782 58.49) (end 65.659 58.4708) (width 0.25) (layer "B.Cu") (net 6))
 (segment (start 59.7916 57.2008) (end 59.7408 57.2008) (width 0.25) (layer "F.Cu") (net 5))
 (segment (start 68.472931 59.517669) (end 70.402331 59.517669) (width 0.25) (layer "F.Cu") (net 5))
 (segment (start 68.472931 59.517669) (end 68.4906 59.5) (width 0.25) (layer "F.Cu") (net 5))
 (segment (start 70.402331 59.517669) (end 70.42 59.5) (width 0.25) (layer "F.Cu") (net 5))
 (segment (start 59.7408 57.2008) (end 56.4416 60.5) (width 0.25) (layer "F.Cu") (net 5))
 (segment (start 56.4416 60.5) (end 54.98 60.5) (width 0.25) (layer "F.Cu") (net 5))
 (segment (start 68.472931 59.517669) (end 68.455262 59.5) (width 0.25) (layer "F.Cu") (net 5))
 (segment (start 70.352331 59.517669) (end 70.37 59.5) (width 0.25) (layer "F.Cu") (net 5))
 (via (at 59.7916 57.2008) (size 0.6) (drill 0.3) (layers "F.Cu" "B.Cu") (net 5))
 (via (at 68.472931 59.517669) (size 0.6) (drill 0.3) (layers "F.Cu" "B.Cu") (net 5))
 (segment (start 61.4492 57.2008) (end 59.7916 57.2008) (width 0.25) (layer "B.Cu") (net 5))
 (segment (start 68.472931 59.517669) (end 65.791469 59.517669) (width 0.25) (layer "B.Cu") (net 5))
 (segment (start 65.791469 59.517669) (end 63.4638 57.19) (width 0.25) (layer "B.Cu") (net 5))
 (segment (start 61.46 57.19) (end 61.4492 57.2008) (width 0.25) (layer "B.Cu") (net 5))
 (segment (start 63.4638 57.19) (end 61.46 57.19) (width 0.25) (layer "B.Cu") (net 5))
 (segment (start 63.627 54.4068) (end 63.1698 54.864) (width 0.25) (layer "F.Cu") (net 9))
 (segment (start 64.5202 65.881) (end 64.5202 66.081) (width 0.25) (layer "F.Cu") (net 9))
 (segment (start 62.8402 65.941) (end 62.8452 65.936) (width 0.25) (layer "F.Cu") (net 9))
 (segment (start 63.5452 65.936) (end 64.4652 65.936) (width 0.25) (layer "F.Cu") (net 9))
 (segment (start 61.6202 65.941) (end 60.4038 65.941) (width 0.25) (layer "F.Cu") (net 9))
 (segment (start 65.6082 68.5546) (end 65.1502 68.0966) (width 0.25) (layer "F.Cu") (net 9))
 (segment (start 58.55 65.1) (end 58.55 65.5858) (width 0.25) (layer "F.Cu") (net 9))
 (segment (start 62.8452 65.936) (end 63.5452 65.936) (width 0.25) (layer "F.Cu") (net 9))
 (segment (start 61.727 52.847) (end 62.1942 52.847) (width 0.25) (layer "F.Cu") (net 9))
 (segment (start 68.5546 68.5292) (end 65.6336 68.5292) (width 0.25) (layer "F.Cu") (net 9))
 (segment (start 65.1502 66.711) (end 65.1502 67.481) (width 0.25) (layer "F.Cu") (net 9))
 (segment (start 68.4754 54.6354) (end 68.83 54.99) (width 0.25) (layer "F.Cu") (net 9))
 (segment (start 63.627 53.497) (end 64.1396 53.497) (width 0.25) (layer "F.Cu") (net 9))
 (segment (start 65.278 54.6354) (end 68.4754 54.6354) (width 0.25) (layer "F.Cu") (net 9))
 (segment (start 62.1942 52.847) (end 62.8442 53.497) (width 0.25) (layer "F.Cu") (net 9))
 (segment (start 64.5202 66.081) (end 65.1502 66.711) (width 0.25) (layer "F.Cu") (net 9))
 (segment (start 61.6202 65.941) (end 62.8402 65.941) (width 0.25) (layer "F.Cu") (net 9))
 (segment (start 59.5628 65.1) (end 58.55 65.1) (width 0.25) (layer "F.Cu") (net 9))
 (segment (start 65.6336 68.5292) (end 65.6082 68.5546) (width 0.25) (layer "F.Cu") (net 9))
 (segment (start 63.627 53.497) (end 63.627 54.4068) (width 0.25) (layer "F.Cu") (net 9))
 (segment (start 64.1396 53.497) (end 65.278 54.6354) (width 0.25) (layer "F.Cu") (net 9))
 (segment (start 69.9008 67.183) (end 68.5546 68.5292) (width 0.25) (layer "F.Cu") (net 9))
 (segment (start 60.4038 65.941) (end 59.5628 65.1) (width 0.25) (layer "F.Cu") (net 9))
 (segment (start 69.9008 63.881) (end 69.9008 67.183) (width 0.25) (layer "F.Cu") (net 9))
 (segment (start 62.8442 53.497) (end 63.627 53.497) (width 0.25) (layer "F.Cu") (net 9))
 (segment (start 65.1502 68.0966) (end 65.1502 67.481) (width 0.25) (layer "F.Cu") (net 9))
 (segment (start 64.4652 65.936) (end 64.5202 65.881) (width 0.25) (layer "F.Cu") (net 9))
 (via (at 69.9008 63.881) (size 0.6) (drill 0.3) (layers "F.Cu" "B.Cu") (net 9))
 (via (at 68.83 54.99) (size 0.6) (drill 0.3) (layers "F.Cu" "B.Cu") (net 9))
 (segment (start 69.9008 56.0832) (end 68.83 55.0124) (width 0.25) (layer "B.Cu") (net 9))
 (segment (start 68.83 55.0124) (end 68.83 54.99) (width 0.25) (layer "B.Cu") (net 9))
 (segment (start 69.9008 63.881) (end 69.9008 56.0832) (width 0.25) (layer "B.Cu") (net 9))
 (segment (start 68.426 63.981) (end 68.4276 63.9826) (width 0.25) (layer "F.Cu") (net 1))
 (segment (start 66.7952 63.981) (end 66.7952 62.8252) (width 0.25) (layer "F.Cu") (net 1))
 (segment (start 66.7952 62.8252) (end 62.7 58.73) (width 0.25) (layer "F.Cu") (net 1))
 (segment (start 62.7 58.73) (end 63.02 58.73) (width 0.25) (layer "F.Cu") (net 1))
 (segment (start 66.7952 63.981) (end 68.426 63.981) (width 0.25) (layer "F.Cu") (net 1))
 (segment (start 57.6 62.56) (end 58.89 61.27) (width 0.25) (layer "F.Cu") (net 2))
 (segment (start 57.6 63.225) (end 57.6 62.56) (width 0.25) (layer "F.Cu") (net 2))
 (segment (start 58.89 61.27) (end 62.7 61.27) (width 0.25) (layer "F.Cu") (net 2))
 (segment (start 62.0058 63.225) (end 59.5 63.225) (width 0.25) (layer "F.Cu") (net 8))
 (segment (start 59.545 63.18) (end 59.5 63.225) (width 0.25) (layer "F.Cu") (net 8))
 (segment (start 64.5202 63.981) (end 62.7618 63.981) (width 0.25) (layer "F.Cu") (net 8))
 (segment (start 62.7618 63.981) (end 62.0058 63.225) (width 0.25) (layer "F.Cu") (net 8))
 (segment (start 66.7952 67.346) (end 66.6602 67.481) (width 0.25) (layer "F.Cu") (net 7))
 (segment (start 67.7164 67.3608) (end 68.4276 67.3608) (width 0.25) (layer "F.Cu") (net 7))
 (segment (start 66.7952 65.881) (end 66.7952 67.196) (width 0.25) (layer "F.Cu") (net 7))
 (segment (start 66.5226 67.481) (end 67.5962 67.481) (width 0.25) (layer "F.Cu") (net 7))
 (segment (start 66.5226 67.481) (end 66.1702 67.481) (width 0.25) (layer "F.Cu") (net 7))
 (segment (start 66.7952 67.196) (end 66.7952 67.346) (width 0.25) (layer "F.Cu") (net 7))
 (segment (start 66.6602 67.481) (end 66.5226 67.481) (width 0.25) (layer "F.Cu") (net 7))
 (segment (start 67.5962 67.481) (end 67.7164 67.3608) (width 0.25) (layer "F.Cu") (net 7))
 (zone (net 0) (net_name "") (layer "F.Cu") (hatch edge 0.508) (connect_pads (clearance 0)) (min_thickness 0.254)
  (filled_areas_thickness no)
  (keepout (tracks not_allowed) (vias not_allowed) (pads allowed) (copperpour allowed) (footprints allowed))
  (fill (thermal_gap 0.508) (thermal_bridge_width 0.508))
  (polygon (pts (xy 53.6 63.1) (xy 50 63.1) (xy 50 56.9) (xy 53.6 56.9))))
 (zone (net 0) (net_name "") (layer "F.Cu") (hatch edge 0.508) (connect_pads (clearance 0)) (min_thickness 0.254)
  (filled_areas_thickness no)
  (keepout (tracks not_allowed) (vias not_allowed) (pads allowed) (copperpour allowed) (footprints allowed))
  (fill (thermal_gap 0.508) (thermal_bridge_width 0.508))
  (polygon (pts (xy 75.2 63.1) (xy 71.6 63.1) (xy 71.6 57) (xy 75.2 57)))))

